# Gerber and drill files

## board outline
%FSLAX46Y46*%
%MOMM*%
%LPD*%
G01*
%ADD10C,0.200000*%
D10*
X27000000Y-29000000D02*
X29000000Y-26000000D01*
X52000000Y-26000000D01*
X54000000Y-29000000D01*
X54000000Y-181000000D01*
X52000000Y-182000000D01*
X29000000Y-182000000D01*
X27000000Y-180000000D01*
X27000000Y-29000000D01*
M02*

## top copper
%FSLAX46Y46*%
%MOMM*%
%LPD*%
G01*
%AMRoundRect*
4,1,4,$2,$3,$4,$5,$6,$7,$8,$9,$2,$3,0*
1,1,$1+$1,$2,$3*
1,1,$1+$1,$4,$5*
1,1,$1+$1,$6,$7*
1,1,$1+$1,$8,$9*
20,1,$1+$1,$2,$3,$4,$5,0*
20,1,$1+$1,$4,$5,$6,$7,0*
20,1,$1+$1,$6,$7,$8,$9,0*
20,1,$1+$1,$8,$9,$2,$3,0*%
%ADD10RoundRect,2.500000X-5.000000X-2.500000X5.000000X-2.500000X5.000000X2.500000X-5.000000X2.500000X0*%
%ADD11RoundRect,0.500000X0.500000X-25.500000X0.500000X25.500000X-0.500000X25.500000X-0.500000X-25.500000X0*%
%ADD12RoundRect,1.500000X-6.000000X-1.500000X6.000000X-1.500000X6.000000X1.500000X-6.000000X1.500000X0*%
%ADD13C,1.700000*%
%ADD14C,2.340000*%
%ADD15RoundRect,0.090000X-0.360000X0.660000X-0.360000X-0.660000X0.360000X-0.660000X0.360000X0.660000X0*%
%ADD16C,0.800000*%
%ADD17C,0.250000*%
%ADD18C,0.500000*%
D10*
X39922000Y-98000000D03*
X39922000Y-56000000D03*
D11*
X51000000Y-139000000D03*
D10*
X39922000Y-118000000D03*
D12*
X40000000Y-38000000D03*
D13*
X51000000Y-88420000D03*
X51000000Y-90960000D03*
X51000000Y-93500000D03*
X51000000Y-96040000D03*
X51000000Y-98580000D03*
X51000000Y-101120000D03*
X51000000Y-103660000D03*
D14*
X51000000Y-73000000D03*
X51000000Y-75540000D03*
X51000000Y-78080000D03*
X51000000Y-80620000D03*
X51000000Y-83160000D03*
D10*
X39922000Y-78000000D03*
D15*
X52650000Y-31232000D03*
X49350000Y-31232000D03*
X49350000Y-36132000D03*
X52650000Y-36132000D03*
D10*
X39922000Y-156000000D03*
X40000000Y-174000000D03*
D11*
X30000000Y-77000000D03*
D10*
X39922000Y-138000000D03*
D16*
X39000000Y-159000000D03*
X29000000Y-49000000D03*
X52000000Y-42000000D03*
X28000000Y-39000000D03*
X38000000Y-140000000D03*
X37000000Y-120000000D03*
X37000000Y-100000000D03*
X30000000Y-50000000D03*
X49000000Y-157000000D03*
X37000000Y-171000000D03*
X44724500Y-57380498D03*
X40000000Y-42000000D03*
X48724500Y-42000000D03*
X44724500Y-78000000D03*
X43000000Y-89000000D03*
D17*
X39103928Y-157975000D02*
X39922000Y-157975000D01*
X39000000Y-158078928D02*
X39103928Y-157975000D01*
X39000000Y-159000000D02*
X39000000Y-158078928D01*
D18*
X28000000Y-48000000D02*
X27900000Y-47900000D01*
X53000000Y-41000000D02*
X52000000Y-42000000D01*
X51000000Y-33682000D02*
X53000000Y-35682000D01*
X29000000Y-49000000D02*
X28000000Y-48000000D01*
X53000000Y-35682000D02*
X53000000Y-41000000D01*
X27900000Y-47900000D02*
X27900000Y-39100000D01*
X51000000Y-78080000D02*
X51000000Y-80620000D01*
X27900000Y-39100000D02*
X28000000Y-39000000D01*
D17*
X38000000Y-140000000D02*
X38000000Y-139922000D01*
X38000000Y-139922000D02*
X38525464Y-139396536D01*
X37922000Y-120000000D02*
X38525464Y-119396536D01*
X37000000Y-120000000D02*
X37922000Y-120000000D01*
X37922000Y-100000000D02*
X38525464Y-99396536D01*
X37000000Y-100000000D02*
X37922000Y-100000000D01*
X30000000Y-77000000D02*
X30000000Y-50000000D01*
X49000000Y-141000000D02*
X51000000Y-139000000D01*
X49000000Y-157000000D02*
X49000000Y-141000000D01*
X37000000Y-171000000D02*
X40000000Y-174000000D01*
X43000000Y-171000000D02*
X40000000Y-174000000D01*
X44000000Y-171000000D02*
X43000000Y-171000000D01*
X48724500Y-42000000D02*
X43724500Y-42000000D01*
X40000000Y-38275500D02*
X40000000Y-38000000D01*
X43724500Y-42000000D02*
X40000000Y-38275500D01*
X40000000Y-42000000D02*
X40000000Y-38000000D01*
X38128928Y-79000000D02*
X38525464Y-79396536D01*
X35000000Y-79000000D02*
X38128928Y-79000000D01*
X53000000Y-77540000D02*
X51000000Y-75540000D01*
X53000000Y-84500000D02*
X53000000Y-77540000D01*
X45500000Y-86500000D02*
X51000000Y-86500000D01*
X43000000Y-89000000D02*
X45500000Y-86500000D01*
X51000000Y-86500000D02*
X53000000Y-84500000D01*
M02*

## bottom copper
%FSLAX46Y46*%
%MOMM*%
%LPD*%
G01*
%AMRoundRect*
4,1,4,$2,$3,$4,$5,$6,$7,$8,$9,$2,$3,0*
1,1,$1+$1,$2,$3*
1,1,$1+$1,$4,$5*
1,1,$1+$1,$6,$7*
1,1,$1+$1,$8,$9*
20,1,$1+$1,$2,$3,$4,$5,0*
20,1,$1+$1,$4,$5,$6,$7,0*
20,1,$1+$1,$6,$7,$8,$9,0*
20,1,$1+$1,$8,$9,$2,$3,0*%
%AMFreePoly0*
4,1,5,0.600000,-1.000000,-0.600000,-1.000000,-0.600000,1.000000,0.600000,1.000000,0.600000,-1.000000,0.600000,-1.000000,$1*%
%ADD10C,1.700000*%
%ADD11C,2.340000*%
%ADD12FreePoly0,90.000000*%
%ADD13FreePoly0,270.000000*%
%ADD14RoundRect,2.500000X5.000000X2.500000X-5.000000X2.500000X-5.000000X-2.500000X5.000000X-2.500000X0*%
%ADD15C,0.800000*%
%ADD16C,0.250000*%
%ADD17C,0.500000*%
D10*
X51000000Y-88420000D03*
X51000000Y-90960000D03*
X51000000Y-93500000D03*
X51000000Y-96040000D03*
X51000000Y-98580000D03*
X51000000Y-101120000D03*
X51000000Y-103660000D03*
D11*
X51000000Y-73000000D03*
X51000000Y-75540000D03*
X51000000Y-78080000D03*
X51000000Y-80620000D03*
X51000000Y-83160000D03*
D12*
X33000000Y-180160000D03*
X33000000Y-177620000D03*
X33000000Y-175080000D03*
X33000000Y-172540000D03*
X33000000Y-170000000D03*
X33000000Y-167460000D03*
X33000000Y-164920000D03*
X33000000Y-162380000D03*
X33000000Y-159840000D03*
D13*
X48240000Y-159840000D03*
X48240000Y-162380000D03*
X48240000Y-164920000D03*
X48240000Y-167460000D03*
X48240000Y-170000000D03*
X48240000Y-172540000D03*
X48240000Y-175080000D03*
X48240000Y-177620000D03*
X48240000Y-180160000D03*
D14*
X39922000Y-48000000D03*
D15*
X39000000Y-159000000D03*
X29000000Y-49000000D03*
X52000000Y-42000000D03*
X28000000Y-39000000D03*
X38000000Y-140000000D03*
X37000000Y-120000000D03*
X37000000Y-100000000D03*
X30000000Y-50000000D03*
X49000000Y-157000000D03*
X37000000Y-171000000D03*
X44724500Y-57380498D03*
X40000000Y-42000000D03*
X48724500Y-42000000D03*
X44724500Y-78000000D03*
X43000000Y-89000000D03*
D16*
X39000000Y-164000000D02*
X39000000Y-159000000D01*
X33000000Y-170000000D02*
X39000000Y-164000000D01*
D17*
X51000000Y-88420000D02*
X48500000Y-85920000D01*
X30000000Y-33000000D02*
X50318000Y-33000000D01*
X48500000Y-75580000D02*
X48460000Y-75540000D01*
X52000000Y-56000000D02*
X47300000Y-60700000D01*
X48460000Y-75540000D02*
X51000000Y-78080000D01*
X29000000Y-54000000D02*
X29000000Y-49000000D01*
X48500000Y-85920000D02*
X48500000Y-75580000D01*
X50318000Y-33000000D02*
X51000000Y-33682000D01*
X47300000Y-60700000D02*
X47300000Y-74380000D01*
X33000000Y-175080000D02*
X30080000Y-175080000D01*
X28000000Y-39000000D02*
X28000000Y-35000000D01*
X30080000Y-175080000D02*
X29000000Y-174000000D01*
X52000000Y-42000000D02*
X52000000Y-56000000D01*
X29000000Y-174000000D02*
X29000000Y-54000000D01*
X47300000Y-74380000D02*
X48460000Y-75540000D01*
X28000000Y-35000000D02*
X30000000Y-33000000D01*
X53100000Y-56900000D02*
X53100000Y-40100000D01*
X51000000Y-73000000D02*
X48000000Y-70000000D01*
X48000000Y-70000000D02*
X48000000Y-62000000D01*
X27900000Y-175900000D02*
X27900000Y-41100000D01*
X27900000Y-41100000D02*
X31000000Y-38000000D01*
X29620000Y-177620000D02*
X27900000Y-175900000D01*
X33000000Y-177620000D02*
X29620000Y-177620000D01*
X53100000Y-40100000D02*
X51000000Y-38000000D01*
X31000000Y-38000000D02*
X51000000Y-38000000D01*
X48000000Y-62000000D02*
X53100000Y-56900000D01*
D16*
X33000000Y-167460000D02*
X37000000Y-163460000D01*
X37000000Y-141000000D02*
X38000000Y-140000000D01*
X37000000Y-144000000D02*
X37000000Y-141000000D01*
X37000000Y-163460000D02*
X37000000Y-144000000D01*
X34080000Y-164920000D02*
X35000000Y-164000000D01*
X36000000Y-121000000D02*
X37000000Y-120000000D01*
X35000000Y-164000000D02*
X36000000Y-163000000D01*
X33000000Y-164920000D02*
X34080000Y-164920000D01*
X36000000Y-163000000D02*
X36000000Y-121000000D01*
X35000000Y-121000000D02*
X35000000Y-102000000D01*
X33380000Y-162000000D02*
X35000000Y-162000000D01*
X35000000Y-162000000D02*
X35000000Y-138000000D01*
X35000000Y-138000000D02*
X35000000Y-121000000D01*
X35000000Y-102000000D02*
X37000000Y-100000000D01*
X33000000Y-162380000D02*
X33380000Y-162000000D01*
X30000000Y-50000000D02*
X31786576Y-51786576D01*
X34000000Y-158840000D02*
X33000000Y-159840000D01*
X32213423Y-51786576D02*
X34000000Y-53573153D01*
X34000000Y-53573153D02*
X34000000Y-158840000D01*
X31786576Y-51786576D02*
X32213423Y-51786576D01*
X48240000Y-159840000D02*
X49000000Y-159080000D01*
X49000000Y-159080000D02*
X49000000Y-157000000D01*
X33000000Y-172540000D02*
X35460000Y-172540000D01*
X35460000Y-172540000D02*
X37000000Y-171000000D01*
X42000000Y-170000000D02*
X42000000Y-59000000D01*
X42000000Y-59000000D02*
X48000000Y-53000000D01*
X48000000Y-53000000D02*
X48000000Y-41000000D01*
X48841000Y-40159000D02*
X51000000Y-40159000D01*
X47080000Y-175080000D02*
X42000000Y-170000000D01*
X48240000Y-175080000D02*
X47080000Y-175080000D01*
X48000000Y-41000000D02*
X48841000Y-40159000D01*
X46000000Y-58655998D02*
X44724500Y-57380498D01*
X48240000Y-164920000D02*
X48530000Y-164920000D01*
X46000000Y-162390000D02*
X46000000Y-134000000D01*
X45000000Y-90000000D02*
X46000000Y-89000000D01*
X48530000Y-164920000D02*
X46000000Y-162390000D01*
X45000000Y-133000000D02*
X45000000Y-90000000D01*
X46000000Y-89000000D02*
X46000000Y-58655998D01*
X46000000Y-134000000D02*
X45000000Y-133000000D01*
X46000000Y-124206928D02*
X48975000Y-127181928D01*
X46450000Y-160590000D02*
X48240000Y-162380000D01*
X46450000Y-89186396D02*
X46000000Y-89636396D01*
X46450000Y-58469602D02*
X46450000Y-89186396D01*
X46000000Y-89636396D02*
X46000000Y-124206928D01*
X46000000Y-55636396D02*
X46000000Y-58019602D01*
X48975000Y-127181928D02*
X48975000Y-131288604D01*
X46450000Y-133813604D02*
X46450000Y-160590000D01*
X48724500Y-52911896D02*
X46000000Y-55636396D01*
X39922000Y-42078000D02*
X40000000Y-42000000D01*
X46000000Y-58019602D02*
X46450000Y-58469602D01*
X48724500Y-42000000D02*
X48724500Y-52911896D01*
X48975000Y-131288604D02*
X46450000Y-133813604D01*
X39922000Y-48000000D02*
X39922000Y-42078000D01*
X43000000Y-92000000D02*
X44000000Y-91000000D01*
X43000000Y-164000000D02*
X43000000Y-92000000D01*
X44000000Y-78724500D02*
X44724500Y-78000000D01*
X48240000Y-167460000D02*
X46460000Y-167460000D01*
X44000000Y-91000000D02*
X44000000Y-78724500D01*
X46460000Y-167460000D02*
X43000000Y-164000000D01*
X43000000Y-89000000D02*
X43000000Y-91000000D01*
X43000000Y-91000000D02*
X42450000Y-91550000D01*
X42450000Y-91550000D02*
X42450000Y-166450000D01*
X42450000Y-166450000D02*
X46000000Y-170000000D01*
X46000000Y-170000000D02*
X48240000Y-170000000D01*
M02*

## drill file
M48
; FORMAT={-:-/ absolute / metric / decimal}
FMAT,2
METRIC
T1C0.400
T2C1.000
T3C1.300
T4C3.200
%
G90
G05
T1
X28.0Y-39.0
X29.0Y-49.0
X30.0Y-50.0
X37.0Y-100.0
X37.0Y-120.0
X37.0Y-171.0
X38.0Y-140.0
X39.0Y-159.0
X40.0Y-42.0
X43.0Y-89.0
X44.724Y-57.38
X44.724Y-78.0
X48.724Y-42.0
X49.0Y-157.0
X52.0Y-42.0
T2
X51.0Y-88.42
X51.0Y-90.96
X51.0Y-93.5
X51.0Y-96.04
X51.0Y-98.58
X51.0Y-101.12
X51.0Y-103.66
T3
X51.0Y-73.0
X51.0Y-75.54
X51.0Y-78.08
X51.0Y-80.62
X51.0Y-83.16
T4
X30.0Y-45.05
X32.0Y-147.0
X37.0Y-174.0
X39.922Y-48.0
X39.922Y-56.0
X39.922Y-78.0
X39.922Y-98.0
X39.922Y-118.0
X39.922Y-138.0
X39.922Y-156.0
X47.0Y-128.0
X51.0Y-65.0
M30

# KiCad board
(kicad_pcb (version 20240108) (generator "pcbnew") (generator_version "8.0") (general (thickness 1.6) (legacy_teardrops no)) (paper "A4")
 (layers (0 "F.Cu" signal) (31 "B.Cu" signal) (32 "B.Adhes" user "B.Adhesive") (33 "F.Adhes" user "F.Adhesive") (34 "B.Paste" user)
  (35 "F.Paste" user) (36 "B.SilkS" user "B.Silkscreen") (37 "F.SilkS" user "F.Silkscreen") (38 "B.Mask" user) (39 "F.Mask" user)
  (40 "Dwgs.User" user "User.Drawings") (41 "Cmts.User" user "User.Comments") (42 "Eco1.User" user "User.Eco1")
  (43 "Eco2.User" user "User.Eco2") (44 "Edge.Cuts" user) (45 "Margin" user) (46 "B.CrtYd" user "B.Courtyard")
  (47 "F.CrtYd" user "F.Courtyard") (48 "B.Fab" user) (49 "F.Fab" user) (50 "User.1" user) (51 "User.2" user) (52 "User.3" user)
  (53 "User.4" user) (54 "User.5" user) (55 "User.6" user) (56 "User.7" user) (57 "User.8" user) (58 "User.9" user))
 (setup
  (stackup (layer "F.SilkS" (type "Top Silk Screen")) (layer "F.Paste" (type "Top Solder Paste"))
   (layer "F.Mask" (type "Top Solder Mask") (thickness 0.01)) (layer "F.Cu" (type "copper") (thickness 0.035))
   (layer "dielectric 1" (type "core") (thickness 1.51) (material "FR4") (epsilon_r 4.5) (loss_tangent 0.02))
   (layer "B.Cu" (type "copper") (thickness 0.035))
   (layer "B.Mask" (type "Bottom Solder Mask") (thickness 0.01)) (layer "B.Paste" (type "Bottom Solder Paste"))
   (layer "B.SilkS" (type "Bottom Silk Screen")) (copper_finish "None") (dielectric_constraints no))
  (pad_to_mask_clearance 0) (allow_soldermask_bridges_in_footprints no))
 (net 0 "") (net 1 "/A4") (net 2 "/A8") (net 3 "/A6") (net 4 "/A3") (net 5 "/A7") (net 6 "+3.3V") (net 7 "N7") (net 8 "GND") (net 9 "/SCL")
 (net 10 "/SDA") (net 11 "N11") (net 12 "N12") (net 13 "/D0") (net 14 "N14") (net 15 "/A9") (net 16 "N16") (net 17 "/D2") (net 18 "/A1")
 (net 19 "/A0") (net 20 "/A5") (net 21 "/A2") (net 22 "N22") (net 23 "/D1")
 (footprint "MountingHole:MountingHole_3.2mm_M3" (layer "F.Cu") (at 37 174)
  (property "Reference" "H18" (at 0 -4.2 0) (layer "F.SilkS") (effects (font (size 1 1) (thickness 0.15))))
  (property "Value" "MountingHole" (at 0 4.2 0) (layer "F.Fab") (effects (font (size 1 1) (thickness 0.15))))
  (pad "" np_thru_hole circle (at 0 0) (size 3.2 3.2) (drill 3.2) (layers "*.Cu" "*.Mask")))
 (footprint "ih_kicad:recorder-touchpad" (layer "F.Cu") (at 39.922 98)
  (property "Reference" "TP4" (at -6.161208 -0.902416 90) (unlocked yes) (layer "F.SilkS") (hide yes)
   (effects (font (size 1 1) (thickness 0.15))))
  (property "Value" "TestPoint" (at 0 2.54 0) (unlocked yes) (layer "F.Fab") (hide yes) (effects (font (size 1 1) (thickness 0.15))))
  (pad "1" smd roundrect (at 0 0) (size 15 10) (layers "F.Cu" "F.Mask") (roundrect_rratio 0.25) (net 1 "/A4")))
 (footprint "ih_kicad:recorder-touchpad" (layer "F.Cu") (at 39.922 56)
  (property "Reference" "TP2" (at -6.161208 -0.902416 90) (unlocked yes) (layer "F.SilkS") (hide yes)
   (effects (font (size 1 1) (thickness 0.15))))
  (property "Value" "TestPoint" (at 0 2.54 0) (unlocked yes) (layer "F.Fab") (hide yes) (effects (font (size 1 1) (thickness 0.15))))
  (pad "1" smd roundrect (at 0 0) (size 15 10) (layers "F.Cu" "F.Mask") (roundrect_rratio 0.25) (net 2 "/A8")))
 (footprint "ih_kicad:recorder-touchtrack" (layer "F.Cu") (at 51 139 90)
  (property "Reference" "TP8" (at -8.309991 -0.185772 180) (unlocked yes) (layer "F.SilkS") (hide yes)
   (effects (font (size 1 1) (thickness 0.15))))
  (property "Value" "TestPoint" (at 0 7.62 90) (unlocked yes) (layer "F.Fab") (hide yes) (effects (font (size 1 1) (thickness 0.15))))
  (pad "1" smd roundrect (at 0 0 90) (size 52 2) (layers "F.Cu" "F.Mask") (roundrect_rratio 0.25) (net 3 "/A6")))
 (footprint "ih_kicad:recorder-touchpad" (layer "F.Cu") (at 39.922 118)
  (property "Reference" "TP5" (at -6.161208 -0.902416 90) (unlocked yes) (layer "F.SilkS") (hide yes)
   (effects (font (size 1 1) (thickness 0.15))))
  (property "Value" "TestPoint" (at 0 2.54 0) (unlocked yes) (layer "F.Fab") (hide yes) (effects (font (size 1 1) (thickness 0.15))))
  (pad "1" smd roundrect (at 0 0) (size 15 10) (layers "F.Cu" "F.Mask") (roundrect_rratio 0.25) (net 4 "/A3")))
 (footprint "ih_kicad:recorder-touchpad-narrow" (layer "F.Cu") (at 40 38)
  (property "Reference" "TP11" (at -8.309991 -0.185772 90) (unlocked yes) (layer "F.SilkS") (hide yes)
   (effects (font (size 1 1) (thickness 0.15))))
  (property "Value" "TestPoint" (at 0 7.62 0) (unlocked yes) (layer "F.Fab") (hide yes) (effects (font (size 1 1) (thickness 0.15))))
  (pad "1" smd roundrect (at 0 0) (size 15 6) (layers "F.Cu" "F.Mask") (roundrect_rratio 0.25) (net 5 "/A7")))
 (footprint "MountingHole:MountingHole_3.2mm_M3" (layer "F.Cu") (at 39.922 118)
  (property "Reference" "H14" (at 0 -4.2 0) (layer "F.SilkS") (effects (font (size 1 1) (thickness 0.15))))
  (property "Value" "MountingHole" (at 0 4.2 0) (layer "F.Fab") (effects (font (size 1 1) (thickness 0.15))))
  (pad "" np_thru_hole circle (at 0 0) (size 3.2 3.2) (drill 3.2) (layers "*.Cu" "*.Mask")))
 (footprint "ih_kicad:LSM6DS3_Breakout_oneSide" (layer "F.Cu") (at 45.92 96.04 -90)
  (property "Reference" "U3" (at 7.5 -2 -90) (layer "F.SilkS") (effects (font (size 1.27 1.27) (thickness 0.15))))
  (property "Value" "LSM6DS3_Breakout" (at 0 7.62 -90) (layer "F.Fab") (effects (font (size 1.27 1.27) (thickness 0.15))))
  (pad "1" thru_hole circle (at -7.62 -5.08 270) (size 1.7 1.7) (drill 1) (layers "*.Cu" "*.Mask") (remove_unused_layers no) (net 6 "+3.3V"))
  (pad "2" thru_hole circle (at -5.08 -5.08 270) (size 1.7 1.7) (drill 1) (layers "*.Cu" "*.Mask") (remove_unused_layers no) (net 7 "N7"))
  (pad "3" thru_hole circle (at -2.54 -5.08 270) (size 1.7 1.7) (drill 1) (layers "*.Cu" "*.Mask") (remove_unused_layers no) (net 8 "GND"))
  (pad "4" thru_hole circle (at 0 -5.08 270) (size 1.7 1.7) (drill 1) (layers "*.Cu" "*.Mask") (remove_unused_layers no) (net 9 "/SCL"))
  (pad "5" thru_hole circle (at 2.54 -5.08 270) (size 1.7 1.7) (drill 1) (layers "*.Cu" "*.Mask") (remove_unused_layers no) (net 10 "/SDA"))
  (pad "6" thru_hole circle (at 5.08 -5.08 270) (size 1.7 1.7) (drill 1) (layers "*.Cu" "*.Mask") (remove_unused_layers no) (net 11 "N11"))
  (pad "7" thru_hole circle (at 7.62 -5.08 270) (size 1.7 1.7) (drill 1) (layers "*.Cu" "*.Mask") (remove_unused_layers no) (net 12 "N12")))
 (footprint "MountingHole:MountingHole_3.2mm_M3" (layer "F.Cu") (at 39.922 48)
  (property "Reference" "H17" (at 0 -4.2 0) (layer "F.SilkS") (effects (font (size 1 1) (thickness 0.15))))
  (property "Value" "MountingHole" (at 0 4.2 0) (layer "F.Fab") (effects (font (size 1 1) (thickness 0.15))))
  (pad "" np_thru_hole circle (at 0 0) (size 3.2 3.2) (drill 3.2) (layers "*.Cu" "*.Mask")))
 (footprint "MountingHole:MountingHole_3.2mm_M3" (layer "F.Cu") (at 39.922 98)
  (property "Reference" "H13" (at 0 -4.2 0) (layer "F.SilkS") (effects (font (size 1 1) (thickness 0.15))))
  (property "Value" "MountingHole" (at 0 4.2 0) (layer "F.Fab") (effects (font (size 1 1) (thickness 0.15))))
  (pad "" np_thru_hole circle (at 0 0) (size 3.2 3.2) (drill 3.2) (layers "*.Cu" "*.Mask")))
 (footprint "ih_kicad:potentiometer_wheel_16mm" (layer "F.Cu") (at 51 73 180)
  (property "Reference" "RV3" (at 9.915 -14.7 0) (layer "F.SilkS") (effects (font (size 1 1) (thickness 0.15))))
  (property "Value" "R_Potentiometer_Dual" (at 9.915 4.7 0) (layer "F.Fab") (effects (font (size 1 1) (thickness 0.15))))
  (pad "1" thru_hole circle (at 0 0 180) (size 2.34 2.34) (drill 1.3) (layers "*.Cu" "*.Mask") (remove_unused_layers no) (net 8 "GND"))
  (pad "2" thru_hole circle (at 0 -2.54 180) (size 2.34 2.34) (drill 1.3) (layers "*.Cu" "*.Mask") (remove_unused_layers no) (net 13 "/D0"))
  (pad "3" thru_hole circle (at 0 -5.08 180) (size 2.34 2.34) (drill 1.3) (layers "*.Cu" "*.Mask") (remove_unused_layers no) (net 6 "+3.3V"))
  (pad "4" thru_hole circle (at 0 -7.62 180) (size 2.34 2.34) (drill 1.3) (layers "*.Cu" "*.Mask") (remove_unused_layers no) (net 6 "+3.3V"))
  (pad "5" thru_hole circle (at 0 -10.16 180) (size 2.34 2.34) (drill 1.3) (layers "*.Cu" "*.Mask") (remove_unused_layers no) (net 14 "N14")))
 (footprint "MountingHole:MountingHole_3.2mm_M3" (layer "F.Cu") (at 39.922 156)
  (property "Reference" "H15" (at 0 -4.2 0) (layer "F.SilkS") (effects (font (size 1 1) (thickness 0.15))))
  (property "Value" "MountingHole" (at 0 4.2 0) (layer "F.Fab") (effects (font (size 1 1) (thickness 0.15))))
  (pad "" np_thru_hole circle (at 0 0) (size 3.2 3.2) (drill 3.2) (layers "*.Cu" "*.Mask")))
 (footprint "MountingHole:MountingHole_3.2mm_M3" (layer "F.Cu") (at 39.922 138)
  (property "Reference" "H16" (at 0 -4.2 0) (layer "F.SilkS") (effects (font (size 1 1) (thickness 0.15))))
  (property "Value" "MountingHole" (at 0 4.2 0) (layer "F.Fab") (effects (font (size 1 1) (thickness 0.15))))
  (pad "" np_thru_hole circle (at 0 0) (size 3.2 3.2) (drill 3.2) (layers "*.Cu" "*.Mask")))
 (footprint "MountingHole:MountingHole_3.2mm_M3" (layer "F.Cu") (at 47 128)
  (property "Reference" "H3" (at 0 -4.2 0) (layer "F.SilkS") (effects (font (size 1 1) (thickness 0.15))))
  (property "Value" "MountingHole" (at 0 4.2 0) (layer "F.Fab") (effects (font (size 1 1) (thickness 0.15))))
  (pad "" np_thru_hole circle (at 0 0) (size 3.2 3.2) (drill 3.2) (layers "*.Cu" "*.Mask")))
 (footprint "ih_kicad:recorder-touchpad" (layer "F.Cu") (at 39.922 78)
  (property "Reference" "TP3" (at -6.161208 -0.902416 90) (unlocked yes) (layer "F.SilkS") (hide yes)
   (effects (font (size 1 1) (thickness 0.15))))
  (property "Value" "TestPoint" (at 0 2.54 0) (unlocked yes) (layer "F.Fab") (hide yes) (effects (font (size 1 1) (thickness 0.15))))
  (pad "1" smd roundrect (at 0 0) (size 15 10) (layers "F.Cu" "F.Mask") (roundrect_rratio 0.25) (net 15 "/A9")))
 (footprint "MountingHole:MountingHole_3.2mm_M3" (layer "F.Cu") (at 30 45.05)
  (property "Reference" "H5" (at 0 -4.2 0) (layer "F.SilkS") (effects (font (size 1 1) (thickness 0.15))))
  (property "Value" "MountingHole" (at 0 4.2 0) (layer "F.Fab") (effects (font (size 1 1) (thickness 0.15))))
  (pad "" np_thru_hole circle (at 0 0) (size 3.2 3.2) (drill 3.2) (layers "*.Cu" "*.Mask")))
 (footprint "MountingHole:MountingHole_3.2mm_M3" (layer "F.Cu") (at 32 147)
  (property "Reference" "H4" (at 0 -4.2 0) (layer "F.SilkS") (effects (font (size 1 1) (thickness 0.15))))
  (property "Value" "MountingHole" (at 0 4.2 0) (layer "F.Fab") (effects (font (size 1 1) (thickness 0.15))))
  (pad "" np_thru_hole circle (at 0 0) (size 3.2 3.2) (drill 3.2) (layers "*.Cu" "*.Mask")))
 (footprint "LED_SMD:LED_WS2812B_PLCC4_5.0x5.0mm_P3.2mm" (layer "F.Cu") (at 51 33.682 -90)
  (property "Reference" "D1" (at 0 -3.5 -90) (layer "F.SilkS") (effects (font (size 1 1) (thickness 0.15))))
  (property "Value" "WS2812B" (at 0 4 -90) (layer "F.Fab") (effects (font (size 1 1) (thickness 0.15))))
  (pad "1" smd roundrect (at -2.45 -1.65 270) (size 1.5 0.9) (layers "F.Cu" "F.Paste" "F.Mask") (roundrect_rratio 0.1) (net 6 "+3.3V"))
  (pad "2" smd roundrect (at -2.45 1.65 270) (size 1.5 0.9) (layers "F.Cu" "F.Paste" "F.Mask") (roundrect_rratio 0.1) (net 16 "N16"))
  (pad "3" smd roundrect (at 2.45 1.65 270) (size 1.5 0.9) (layers "F.Cu" "F.Paste" "F.Mask") (roundrect_rratio 0.1) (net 8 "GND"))
  (pad "4" smd roundrect (at 2.45 -1.65 270) (size 1.5 0.9) (layers "F.Cu" "F.Paste" "F.Mask") (roundrect_rratio 0.1) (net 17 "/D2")))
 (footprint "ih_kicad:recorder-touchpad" (layer "F.Cu") (at 39.922 156)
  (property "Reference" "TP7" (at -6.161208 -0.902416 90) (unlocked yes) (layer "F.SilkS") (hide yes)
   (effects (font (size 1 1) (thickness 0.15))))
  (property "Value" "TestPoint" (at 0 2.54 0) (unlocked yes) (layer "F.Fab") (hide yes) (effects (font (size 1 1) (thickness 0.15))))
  (pad "1" smd roundrect (at 0 0) (size 15 10) (layers "F.Cu" "F.Mask") (roundrect_rratio 0.25) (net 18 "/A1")))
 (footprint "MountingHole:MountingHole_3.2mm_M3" (layer "F.Cu") (at 39.922 78)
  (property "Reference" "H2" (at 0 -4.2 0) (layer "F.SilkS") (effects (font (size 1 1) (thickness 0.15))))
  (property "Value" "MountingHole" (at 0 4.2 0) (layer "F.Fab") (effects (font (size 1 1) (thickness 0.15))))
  (pad "" np_thru_hole circle (at 0 0) (size 3.2 3.2) (drill 3.2) (layers "*.Cu" "*.Mask")))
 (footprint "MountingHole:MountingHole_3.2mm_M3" (layer "F.Cu") (at 51 65)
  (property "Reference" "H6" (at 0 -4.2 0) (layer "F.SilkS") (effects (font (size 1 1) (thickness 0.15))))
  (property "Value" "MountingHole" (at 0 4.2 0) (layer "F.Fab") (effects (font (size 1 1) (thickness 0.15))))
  (pad "" np_thru_hole circle (at 0 0) (size 3.2 3.2) (drill 3.2) (layers "*.Cu" "*.Mask")))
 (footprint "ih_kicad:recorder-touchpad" (layer "F.Cu") (at 40 174)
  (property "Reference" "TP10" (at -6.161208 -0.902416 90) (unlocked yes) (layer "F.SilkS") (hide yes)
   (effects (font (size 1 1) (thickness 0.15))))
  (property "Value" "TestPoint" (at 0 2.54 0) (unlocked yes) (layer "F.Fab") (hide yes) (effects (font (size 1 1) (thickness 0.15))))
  (pad "1" smd roundrect (at 0 0) (size 15 10) (layers "F.Cu" "F.Mask") (roundrect_rratio 0.25) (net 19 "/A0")))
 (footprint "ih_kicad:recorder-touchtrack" (layer "F.Cu") (at 30 77 90)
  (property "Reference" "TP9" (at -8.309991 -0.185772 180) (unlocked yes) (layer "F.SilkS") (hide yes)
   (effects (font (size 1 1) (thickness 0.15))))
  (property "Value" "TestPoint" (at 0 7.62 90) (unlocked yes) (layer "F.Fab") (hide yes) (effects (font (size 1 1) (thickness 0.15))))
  (pad "1" smd roundrect (at 0 0 90) (size 52 2) (layers "F.Cu" "F.Mask") (roundrect_rratio 0.25) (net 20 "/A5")))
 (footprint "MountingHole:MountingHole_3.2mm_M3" (layer "F.Cu") (at 39.922 56)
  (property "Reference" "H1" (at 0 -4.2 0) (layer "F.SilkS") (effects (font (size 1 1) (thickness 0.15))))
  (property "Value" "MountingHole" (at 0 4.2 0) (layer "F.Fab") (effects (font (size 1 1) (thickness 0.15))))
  (pad "" np_thru_hole circle (at 0 0) (size 3.2 3.2) (drill 3.2) (layers "*.Cu" "*.Mask")))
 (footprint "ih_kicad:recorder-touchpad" (layer "F.Cu") (at 39.922 138)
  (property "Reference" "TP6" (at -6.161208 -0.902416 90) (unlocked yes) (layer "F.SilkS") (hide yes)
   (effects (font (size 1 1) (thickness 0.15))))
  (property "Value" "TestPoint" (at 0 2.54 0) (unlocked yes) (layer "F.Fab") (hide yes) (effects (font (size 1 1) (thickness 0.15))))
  (pad "1" smd roundrect (at 0 0) (size 15 10) (layers "F.Cu" "F.Mask") (roundrect_rratio 0.25) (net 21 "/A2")))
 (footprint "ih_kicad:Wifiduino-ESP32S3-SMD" (layer "B.Cu") (at 40.62 170)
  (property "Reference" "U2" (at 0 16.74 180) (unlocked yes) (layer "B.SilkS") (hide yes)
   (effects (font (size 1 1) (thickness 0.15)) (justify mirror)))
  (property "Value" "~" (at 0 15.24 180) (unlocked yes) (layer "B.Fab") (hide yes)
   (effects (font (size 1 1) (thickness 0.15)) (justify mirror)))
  (pad "1" smd custom (at -7.62 10.16 90) (size 1.2 2) (layers "B.Cu" "B.Paste" "B.Mask") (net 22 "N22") (thermal_bridge_angle 45)
   (options (clearance outline) (anchor rect)) (primitives))
  (pad "2" smd custom (at -7.62 7.62 90) (size 1.2 2) (layers "B.Cu" "B.Paste" "B.Mask") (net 8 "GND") (thermal_bridge_angle 45)
   (options (clearance outline) (anchor rect)) (primitives))
  (pad "3" smd custom (at -7.62 5.08 90) (size 1.2 2) (layers "B.Cu" "B.Paste" "B.Mask") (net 6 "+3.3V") (thermal_bridge_angle 45)
   (options (clearance outline) (anchor rect)) (primitives))
  (pad "4" smd custom (at -7.62 2.54 90) (size 1.2 2) (layers "B.Cu" "B.Paste" "B.Mask") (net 19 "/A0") (thermal_bridge_angle 45)
   (options (clearance outline) (anchor rect)) (primitives))
  (pad "5" smd custom (at -7.62 0 90) (size 1.2 2) (layers "B.Cu" "B.Paste" "B.Mask") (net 18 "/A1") (thermal_bridge_angle 45)
   (options (clearance outline) (anchor rect)) (primitives))
  (pad "6" smd custom (at -7.62 -2.54 90) (size 1.2 2) (layers "B.Cu" "B.Paste" "B.Mask") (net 21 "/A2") (thermal_bridge_angle 45)
   (options (clearance outline) (anchor rect)) (primitives))
  (pad "7" smd custom (at -7.62 -5.08 90) (size 1.2 2) (layers "B.Cu" "B.Paste" "B.Mask") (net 4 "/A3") (thermal_bridge_angle 45)
   (options (clearance outline) (anchor rect)) (primitives))
  (pad "8" smd custom (at -7.62 -7.62 90) (size 1.2 2) (layers "B.Cu" "B.Paste" "B.Mask") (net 1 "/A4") (thermal_bridge_angle 45)
   (options (clearance outline) (anchor rect)) (primitives))
  (pad "9" smd custom (at -7.62 -10.16 90) (size 1.2 2) (layers "B.Cu" "B.Paste" "B.Mask") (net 20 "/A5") (thermal_bridge_angle 45)
   (options (clearance outline) (anchor rect)) (primitives))
  (pad "10" smd custom (at 7.62 -10.16 270) (size 1.2 2) (layers "B.Cu" "B.Paste" "B.Mask") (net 3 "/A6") (thermal_bridge_angle 45)
   (options (clearance outline) (anchor rect)) (primitives))
  (pad "11" smd custom (at 7.62 -7.62 270) (size 1.2 2) (layers "B.Cu" "B.Paste" "B.Mask") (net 5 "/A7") (thermal_bridge_angle 45)
   (options (clearance outline) (anchor rect)) (primitives))
  (pad "12" smd custom (at 7.62 -5.08 270) (size 1.2 2) (layers "B.Cu" "B.Paste" "B.Mask") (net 2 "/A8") (thermal_bridge_angle 45)
   (options (clearance outline) (anchor rect)) (primitives))
  (pad "13" smd custom (at 7.62 -2.54 270) (size 1.2 2) (layers "B.Cu" "B.Paste" "B.Mask") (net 15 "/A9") (thermal_bridge_angle 45)
   (options (clearance outline) (anchor rect)) (primitives))
  (pad "14" smd custom (at 7.62 0 270) (size 1.2 2) (layers "B.Cu" "B.Paste" "B.Mask") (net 13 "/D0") (thermal_bridge_angle 45)
   (options (clearance outline) (anchor rect)) (primitives))
  (pad "15" smd custom (at 7.62 2.54 270) (size 1.2 2) (layers "B.Cu" "B.Paste" "B.Mask") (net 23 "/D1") (thermal_bridge_angle 45)
   (options (clearance outline) (anchor rect)) (primitives))
  (pad "16" smd custom (at 7.62 5.08 270) (size 1.2 2) (layers "B.Cu" "B.Paste" "B.Mask") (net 17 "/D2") (thermal_bridge_angle 45)
   (options (clearance outline) (anchor rect)) (primitives))
  (pad "17" smd custom (at 7.62 7.62 270) (size 1.2 2) (layers "B.Cu" "B.Paste" "B.Mask") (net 10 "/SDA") (thermal_bridge_angle 45)
   (options (clearance outline) (anchor rect)) (primitives))
  (pad "18" smd custom (at 7.62 10.16 270) (size 1.2 2) (layers "B.Cu" "B.Paste" "B.Mask") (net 9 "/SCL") (thermal_bridge_angle 45)
   (options (clearance outline) (anchor rect)) (primitives)))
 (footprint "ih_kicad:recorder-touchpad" (layer "B.Cu") (at 39.922 48 180)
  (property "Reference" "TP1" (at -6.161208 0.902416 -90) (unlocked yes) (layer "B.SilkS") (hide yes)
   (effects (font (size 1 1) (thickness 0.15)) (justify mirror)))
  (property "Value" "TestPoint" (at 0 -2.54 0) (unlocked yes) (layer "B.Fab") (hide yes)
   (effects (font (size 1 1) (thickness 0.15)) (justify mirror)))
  (pad "1" smd roundrect (at 0 0 180) (size 15 10) (layers "B.Cu" "B.Mask") (roundrect_rratio 0.25) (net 5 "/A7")))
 (gr_poly
  (pts (xy 27 29) (xy 29 26) (xy 52 26) (xy 54 29) (xy 54 181) (xy 52 182) (xy 29 182) (xy 27 180)) (stroke (width 0.2) (type solid))
  (fill none) (layer "Edge.Cuts"))
 (segment (start 39.103928 157.975) (end 39.922 157.975) (width 0.25) (layer "F.Cu") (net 18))
 (segment (start 39 158.078928) (end 39.103928 157.975) (width 0.25) (layer "F.Cu") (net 18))
 (segment (start 39 159) (end 39 158.078928) (width 0.25) (layer "F.Cu") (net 18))
 (via (at 39 159) (size 0.8) (drill 0.4) (layers "F.Cu" "B.Cu") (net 18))
 (segment (start 39 164) (end 39 159) (width 0.25) (layer "B.Cu") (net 18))
 (segment (start 33 170) (end 39 164) (width 0.25) (layer "B.Cu") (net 18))
 (segment (start 28 48) (end 27.9 47.9) (width 0.5) (layer "F.Cu") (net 6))
 (segment (start 53 41) (end 52 42) (width 0.5) (layer "F.Cu") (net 6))
 (segment (start 51 33.682) (end 53 35.682) (width 0.5) (layer "F.Cu") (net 6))
 (segment (start 29 49) (end 28 48) (width 0.5) (layer "F.Cu") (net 6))
 (segment (start 53 35.682) (end 53 41) (width 0.5) (layer "F.Cu") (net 6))
 (segment (start 27.9 47.9) (end 27.9 39.1) (width 0.5) (layer "F.Cu") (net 6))
 (segment (start 51 78.08) (end 51 80.62) (width 0.5) (layer "F.Cu") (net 6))
 (segment (start 27.9 39.1) (end 28 39) (width 0.5) (layer "F.Cu") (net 6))
 (via (at 29 49) (size 0.8) (drill 0.4) (layers "F.Cu" "B.Cu") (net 6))
 (via (at 52 42) (size 0.8) (drill 0.4) (layers "F.Cu" "B.Cu") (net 6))
 (via (at 28 39) (size 0.8) (drill 0.4) (layers "F.Cu" "B.Cu") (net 6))
 (segment (start 51 88.42) (end 48.5 85.92) (width 0.5) (layer "B.Cu") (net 6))
 (segment (start 30 33) (end 50.318 33) (width 0.5) (layer "B.Cu") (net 6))
 (segment (start 48.5 75.58) (end 48.46 75.54) (width 0.5) (layer "B.Cu") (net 6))
 (segment (start 52 56) (end 47.3 60.7) (width 0.5) (layer "B.Cu") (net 6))
 (segment (start 48.46 75.54) (end 51 78.08) (width 0.5) (layer "B.Cu") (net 6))
 (segment (start 29 54) (end 29 49) (width 0.5) (layer "B.Cu") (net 6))
 (segment (start 48.5 85.92) (end 48.5 75.58) (width 0.5) (layer "B.Cu") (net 6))
 (segment (start 50.318 33) (end 51 33.682) (width 0.5) (layer "B.Cu") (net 6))
 (segment (start 47.3 60.7) (end 47.3 74.38) (width 0.5) (layer "B.Cu") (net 6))
 (segment (start 33 175.08) (end 30.08 175.08) (width 0.5) (layer "B.Cu") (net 6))
 (segment (start 28 39) (end 28 35) (width 0.5) (layer "B.Cu") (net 6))
 (segment (start 30.08 175.08) (end 29 174) (width 0.5) (layer "B.Cu") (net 6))
 (segment (start 52 42) (end 52 56) (width 0.5) (layer "B.Cu") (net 6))
 (segment (start 29 174) (end 29 54) (width 0.5) (layer "B.Cu") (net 6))
 (segment (start 47.3 74.38) (end 48.46 75.54) (width 0.5) (layer "B.Cu") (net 6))
 (segment (start 28 35) (end 30 33) (width 0.5) (layer "B.Cu") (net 6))
 (segment (start 53.1 56.9) (end 53.1 40.1) (width 0.5) (layer "B.Cu") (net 8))
 (segment (start 51 73) (end 48 70) (width 0.5) (layer "B.Cu") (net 8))
 (segment (start 48 70) (end 48 62) (width 0.5) (layer "B.Cu") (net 8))
 (segment (start 27.9 175.9) (end 27.9 41.1) (width 0.5) (layer "B.Cu") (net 8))
 (segment (start 27.9 41.1) (end 31 38) (width 0.5) (layer "B.Cu") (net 8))
 (segment (start 29.62 177.62) (end 27.9 175.9) (width 0.5) (layer "B.Cu") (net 8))
 (segment (start 33 177.62) (end 29.62 177.62) (width 0.5) (layer "B.Cu") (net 8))
 (segment (start 53.1 40.1) (end 51 38) (width 0.5) (layer "B.Cu") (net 8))
 (segment (start 31 38) (end 51 38) (width 0.5) (layer "B.Cu") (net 8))
 (segment (start 48 62) (end 53.1 56.9) (width 0.5) (layer "B.Cu") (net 8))
 (segment (start 38 140) (end 38 139.922) (width 0.25) (layer "F.Cu") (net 21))
 (segment (start 38 139.922) (end 38.525464 139.396536) (width 0.25) (layer "F.Cu") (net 21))
 (via (at 38 140) (size 0.8) (drill 0.4) (layers "F.Cu" "B.Cu") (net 21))
 (segment (start 33 167.46) (end 37 163.46) (width 0.25) (layer "B.Cu") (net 21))
 (segment (start 37 141) (end 38 140) (width 0.25) (layer "B.Cu") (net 21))
 (segment (start 37 144) (end 37 141) (width 0.25) (layer "B.Cu") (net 21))
 (segment (start 37 163.46) (end 37 144) (width 0.25) (layer "B.Cu") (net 21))
 (segment (start 37.922 120) (end 38.525464 119.396536) (width 0.25) (layer "F.Cu") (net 4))
 (segment (start 37 120) (end 37.922 120) (width 0.25) (layer "F.Cu") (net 4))
 (via (at 37 120) (size 0.8) (drill 0.4) (layers "F.Cu" "B.Cu") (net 4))
 (segment (start 34.08 164.92) (end 35 164) (width 0.25) (layer "B.Cu") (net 4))
 (segment (start 36 121) (end 37 120) (width 0.25) (layer "B.Cu") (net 4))
 (segment (start 35 164) (end 36 163) (width 0.25) (layer "B.Cu") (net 4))
 (segment (start 33 164.92) (end 34.08 164.92) (width 0.25) (layer "B.Cu") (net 4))
 (segment (start 36 163) (end 36 121) (width 0.25) (layer "B.Cu") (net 4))
 (segment (start 37.922 100) (end 38.525464 99.396536) (width 0.25) (layer "F.Cu") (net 1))
 (segment (start 37 100) (end 37.922 100) (width 0.25) (layer "F.Cu") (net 1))
 (via (at 37 100) (size 0.8) (drill 0.4) (layers "F.Cu" "B.Cu") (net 1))
 (segment (start 35 121) (end 35 102) (width 0.25) (layer "B.Cu") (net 1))
 (segment (start 33.38 162) (end 35 162) (width 0.25) (layer "B.Cu") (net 1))
 (segment (start 35 162) (end 35 138) (width 0.25) (layer "B.Cu") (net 1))
 (segment (start 35 138) (end 35 121) (width 0.25) (layer "B.Cu") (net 1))
 (segment (start 35 102) (end 37 100) (width 0.25) (layer "B.Cu") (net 1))
 (segment (start 33 162.38) (end 33.38 162) (width 0.25) (layer "B.Cu") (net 1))
 (segment (start 30 77) (end 30 50) (width 0.25) (layer "F.Cu") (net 20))
 (via (at 30 50) (size 0.8) (drill 0.4) (layers "F.Cu" "B.Cu") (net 20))
 (segment (start 30 50) (end 31.786576 51.786576) (width 0.25) (layer "B.Cu") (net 20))
 (segment (start 34 158.84) (end 33 159.84) (width 0.25) (layer "B.Cu") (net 20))
 (segment (start 32.213423 51.786576) (end 34 53.573153) (width 0.25) (layer "B.Cu") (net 20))
 (segment (start 34 53.573153) (end 34 158.84) (width 0.25) (layer "B.Cu") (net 20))
 (segment (start 31.786576 51.786576) (end 32.213423 51.786576) (width 0.25) (layer "B.Cu") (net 20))
 (segment (start 49 141) (end 51 139) (width 0.25) (layer "F.Cu") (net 3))
 (segment (start 49 157) (end 49 141) (width 0.25) (layer "F.Cu") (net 3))
 (via (at 49 157) (size 0.8) (drill 0.4) (layers "F.Cu" "B.Cu") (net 3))
 (segment (start 48.24 159.84) (end 49 159.08) (width 0.25) (layer "B.Cu") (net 3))
 (segment (start 49 159.08) (end 49 157) (width 0.25) (layer "B.Cu") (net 3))
 (segment (start 37 171) (end 40 174) (width 0.25) (layer "F.Cu") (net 19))
 (segment (start 43 171) (end 40 174) (width 0.25) (layer "F.Cu") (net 19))
 (segment (start 44 171) (end 43 171) (width 0.25) (layer "F.Cu") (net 19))
 (via (at 37 171) (size 0.8) (drill 0.4) (layers "F.Cu" "B.Cu") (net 19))
 (segment (start 33 172.54) (end 35.46 172.54) (width 0.25) (layer "B.Cu") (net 19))
 (segment (start 35.46 172.54) (end 37 171) (width 0.25) (layer "B.Cu") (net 19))
 (segment (start 42 170) (end 42 59) (width 0.25) (layer "B.Cu") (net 17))
 (segment (start 42 59) (end 48 53) (width 0.25) (layer "B.Cu") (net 17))
 (segment (start 48 53) (end 48 41) (width 0.25) (layer "B.Cu") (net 17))
 (segment (start 48.841 40.159) (end 51 40.159) (width 0.25) (layer "B.Cu") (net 17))
 (segment (start 47.08 175.08) (end 42 170) (width 0.25) (layer "B.Cu") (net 17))
 (segment (start 48.24 175.08) (end 47.08 175.08) (width 0.25) (layer "B.Cu") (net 17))
 (segment (start 48 41) (end 48.841 40.159) (width 0.25) (layer "B.Cu") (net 17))
 (via (at 44.7245 57.380498) (size 0.8) (drill 0.4) (layers "F.Cu" "B.Cu") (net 2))
 (segment (start 46 58.655998) (end 44.7245 57.380498) (width 0.25) (layer "B.Cu") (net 2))
 (segment (start 48.24 164.92) (end 48.53 164.92) (width 0.25) (layer "B.Cu") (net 2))
 (segment (start 46 162.39) (end 46 134) (width 0.25) (layer "B.Cu") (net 2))
 (segment (start 45 90) (end 46 89) (width 0.25) (layer "B.Cu") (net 2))
 (segment (start 48.53 164.92) (end 46 162.39) (width 0.25) (layer "B.Cu") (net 2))
 (segment (start 45 133) (end 45 90) (width 0.25) (layer "B.Cu") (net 2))
 (segment (start 46 89) (end 46 58.655998) (width 0.25) (layer "B.Cu") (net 2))
 (segment (start 46 134) (end 45 133) (width 0.25) (layer "B.Cu") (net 2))
 (segment (start 48.7245 42) (end 43.7245 42) (width 0.25) (layer "F.Cu") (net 5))
 (segment (start 40 38.2755) (end 40 38) (width 0.25) (layer "F.Cu") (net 5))
 (segment (start 43.7245 42) (end 40 38.2755) (width 0.25) (layer "F.Cu") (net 5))
 (segment (start 40 42) (end 40 38) (width 0.25) (layer "F.Cu") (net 5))
 (via (at 40 42) (size 0.8) (drill 0.4) (layers "F.Cu" "B.Cu") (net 5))
 (via (at 48.7245 42) (size 0.8) (drill 0.4) (layers "F.Cu" "B.Cu") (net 5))
 (segment (start 46 124.206928) (end 48.975 127.181928) (width 0.25) (layer "B.Cu") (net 5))
 (segment (start 46.45 160.59) (end 48.24 162.38) (width 0.25) (layer "B.Cu") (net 5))
 (segment (start 46.45 89.186396) (end 46 89.636396) (width 0.25) (layer "B.Cu") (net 5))
 (segment (start 46.45 58.469602) (end 46.45 89.186396) (width 0.25) (layer "B.Cu") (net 5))
 (segment (start 46 89.636396) (end 46 124.206928) (width 0.25) (layer "B.Cu") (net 5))
 (segment (start 46 55.636396) (end 46 58.019602) (width 0.25) (layer "B.Cu") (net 5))
 (segment (start 48.975 127.181928) (end 48.975 131.288604) (width 0.25) (layer "B.Cu") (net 5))
 (segment (start 46.45 133.813604) (end 46.45 160.59) (width 0.25) (layer "B.Cu") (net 5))
 (segment (start 48.7245 52.911896) (end 46 55.636396) (width 0.25) (layer "B.Cu") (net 5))
 (segment (start 39.922 42.078) (end 40 42) (width 0.25) (layer "B.Cu") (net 5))
 (segment (start 46 58.019602) (end 46.45 58.469602) (width 0.25) (layer "B.Cu") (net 5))
 (segment (start 48.7245 42) (end 48.7245 52.911896) (width 0.25) (layer "B.Cu") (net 5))
 (segment (start 48.975 131.288604) (end 46.45 133.813604) (width 0.25) (layer "B.Cu") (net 5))
 (segment (start 39.922 48) (end 39.922 42.078) (width 0.25) (layer "B.Cu") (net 5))
 (segment (start 38.128928 79) (end 38.525464 79.396536) (width 0.25) (layer "F.Cu") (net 15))
 (segment (start 35 79) (end 38.128928 79) (width 0.25) (layer "F.Cu") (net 15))
 (via (at 44.7245 78) (size 0.8) (drill 0.4) (layers "F.Cu" "B.Cu") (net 15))
 (segment (start 43 92) (end 44 91) (width 0.25) (layer "B.Cu") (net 15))
 (segment (start 43 164) (end 43 92) (width 0.25) (layer "B.Cu") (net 15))
 (segment (start 44 78.7245) (end 44.7245 78) (width 0.25) (layer "B.Cu") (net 15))
 (segment (start 48.24 167.46) (end 46.46 167.46) (width 0.25) (layer "B.Cu") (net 15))
 (segment (start 44 91) (end 44 78.7245) (width 0.25) (layer "B.Cu") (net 15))
 (segment (start 46.46 167.46) (end 43 164) (width 0.25) (layer "B.Cu") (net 15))
 (segment (start 53 77.54) (end 51 75.54) (width 0.25) (layer "F.Cu") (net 13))
 (segment (start 53 84.5) (end 53 77.54) (width 0.25) (layer "F.Cu") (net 13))
 (segment (start 45.5 86.5) (end 51 86.5) (width 0.25) (layer "F.Cu") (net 13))
 (segment (start 43 89) (end 45.5 86.5) (width 0.25) (layer "F.Cu") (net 13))
 (segment (start 51 86.5) (end 53 84.5) (width 0.25) (layer "F.Cu") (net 13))
 (via (at 43 89) (size 0.8) (drill 0.4) (layers "F.Cu" "B.Cu") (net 13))
 (segment (start 43 89) (end 43 91) (width 0.25) (layer "B.Cu") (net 13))
 (segment (start 43 91) (end 42.45 91.55) (width 0.25) (layer "B.Cu") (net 13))
 (segment (start 42.45 91.55) (end 42.45 166.45) (width 0.25) (layer "B.Cu") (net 13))
 (segment (start 42.45 166.45) (end 46 170) (width 0.25) (layer "B.Cu") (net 13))
 (segment (start 46 170) (end 48.24 170) (width 0.25) (layer "B.Cu") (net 13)))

